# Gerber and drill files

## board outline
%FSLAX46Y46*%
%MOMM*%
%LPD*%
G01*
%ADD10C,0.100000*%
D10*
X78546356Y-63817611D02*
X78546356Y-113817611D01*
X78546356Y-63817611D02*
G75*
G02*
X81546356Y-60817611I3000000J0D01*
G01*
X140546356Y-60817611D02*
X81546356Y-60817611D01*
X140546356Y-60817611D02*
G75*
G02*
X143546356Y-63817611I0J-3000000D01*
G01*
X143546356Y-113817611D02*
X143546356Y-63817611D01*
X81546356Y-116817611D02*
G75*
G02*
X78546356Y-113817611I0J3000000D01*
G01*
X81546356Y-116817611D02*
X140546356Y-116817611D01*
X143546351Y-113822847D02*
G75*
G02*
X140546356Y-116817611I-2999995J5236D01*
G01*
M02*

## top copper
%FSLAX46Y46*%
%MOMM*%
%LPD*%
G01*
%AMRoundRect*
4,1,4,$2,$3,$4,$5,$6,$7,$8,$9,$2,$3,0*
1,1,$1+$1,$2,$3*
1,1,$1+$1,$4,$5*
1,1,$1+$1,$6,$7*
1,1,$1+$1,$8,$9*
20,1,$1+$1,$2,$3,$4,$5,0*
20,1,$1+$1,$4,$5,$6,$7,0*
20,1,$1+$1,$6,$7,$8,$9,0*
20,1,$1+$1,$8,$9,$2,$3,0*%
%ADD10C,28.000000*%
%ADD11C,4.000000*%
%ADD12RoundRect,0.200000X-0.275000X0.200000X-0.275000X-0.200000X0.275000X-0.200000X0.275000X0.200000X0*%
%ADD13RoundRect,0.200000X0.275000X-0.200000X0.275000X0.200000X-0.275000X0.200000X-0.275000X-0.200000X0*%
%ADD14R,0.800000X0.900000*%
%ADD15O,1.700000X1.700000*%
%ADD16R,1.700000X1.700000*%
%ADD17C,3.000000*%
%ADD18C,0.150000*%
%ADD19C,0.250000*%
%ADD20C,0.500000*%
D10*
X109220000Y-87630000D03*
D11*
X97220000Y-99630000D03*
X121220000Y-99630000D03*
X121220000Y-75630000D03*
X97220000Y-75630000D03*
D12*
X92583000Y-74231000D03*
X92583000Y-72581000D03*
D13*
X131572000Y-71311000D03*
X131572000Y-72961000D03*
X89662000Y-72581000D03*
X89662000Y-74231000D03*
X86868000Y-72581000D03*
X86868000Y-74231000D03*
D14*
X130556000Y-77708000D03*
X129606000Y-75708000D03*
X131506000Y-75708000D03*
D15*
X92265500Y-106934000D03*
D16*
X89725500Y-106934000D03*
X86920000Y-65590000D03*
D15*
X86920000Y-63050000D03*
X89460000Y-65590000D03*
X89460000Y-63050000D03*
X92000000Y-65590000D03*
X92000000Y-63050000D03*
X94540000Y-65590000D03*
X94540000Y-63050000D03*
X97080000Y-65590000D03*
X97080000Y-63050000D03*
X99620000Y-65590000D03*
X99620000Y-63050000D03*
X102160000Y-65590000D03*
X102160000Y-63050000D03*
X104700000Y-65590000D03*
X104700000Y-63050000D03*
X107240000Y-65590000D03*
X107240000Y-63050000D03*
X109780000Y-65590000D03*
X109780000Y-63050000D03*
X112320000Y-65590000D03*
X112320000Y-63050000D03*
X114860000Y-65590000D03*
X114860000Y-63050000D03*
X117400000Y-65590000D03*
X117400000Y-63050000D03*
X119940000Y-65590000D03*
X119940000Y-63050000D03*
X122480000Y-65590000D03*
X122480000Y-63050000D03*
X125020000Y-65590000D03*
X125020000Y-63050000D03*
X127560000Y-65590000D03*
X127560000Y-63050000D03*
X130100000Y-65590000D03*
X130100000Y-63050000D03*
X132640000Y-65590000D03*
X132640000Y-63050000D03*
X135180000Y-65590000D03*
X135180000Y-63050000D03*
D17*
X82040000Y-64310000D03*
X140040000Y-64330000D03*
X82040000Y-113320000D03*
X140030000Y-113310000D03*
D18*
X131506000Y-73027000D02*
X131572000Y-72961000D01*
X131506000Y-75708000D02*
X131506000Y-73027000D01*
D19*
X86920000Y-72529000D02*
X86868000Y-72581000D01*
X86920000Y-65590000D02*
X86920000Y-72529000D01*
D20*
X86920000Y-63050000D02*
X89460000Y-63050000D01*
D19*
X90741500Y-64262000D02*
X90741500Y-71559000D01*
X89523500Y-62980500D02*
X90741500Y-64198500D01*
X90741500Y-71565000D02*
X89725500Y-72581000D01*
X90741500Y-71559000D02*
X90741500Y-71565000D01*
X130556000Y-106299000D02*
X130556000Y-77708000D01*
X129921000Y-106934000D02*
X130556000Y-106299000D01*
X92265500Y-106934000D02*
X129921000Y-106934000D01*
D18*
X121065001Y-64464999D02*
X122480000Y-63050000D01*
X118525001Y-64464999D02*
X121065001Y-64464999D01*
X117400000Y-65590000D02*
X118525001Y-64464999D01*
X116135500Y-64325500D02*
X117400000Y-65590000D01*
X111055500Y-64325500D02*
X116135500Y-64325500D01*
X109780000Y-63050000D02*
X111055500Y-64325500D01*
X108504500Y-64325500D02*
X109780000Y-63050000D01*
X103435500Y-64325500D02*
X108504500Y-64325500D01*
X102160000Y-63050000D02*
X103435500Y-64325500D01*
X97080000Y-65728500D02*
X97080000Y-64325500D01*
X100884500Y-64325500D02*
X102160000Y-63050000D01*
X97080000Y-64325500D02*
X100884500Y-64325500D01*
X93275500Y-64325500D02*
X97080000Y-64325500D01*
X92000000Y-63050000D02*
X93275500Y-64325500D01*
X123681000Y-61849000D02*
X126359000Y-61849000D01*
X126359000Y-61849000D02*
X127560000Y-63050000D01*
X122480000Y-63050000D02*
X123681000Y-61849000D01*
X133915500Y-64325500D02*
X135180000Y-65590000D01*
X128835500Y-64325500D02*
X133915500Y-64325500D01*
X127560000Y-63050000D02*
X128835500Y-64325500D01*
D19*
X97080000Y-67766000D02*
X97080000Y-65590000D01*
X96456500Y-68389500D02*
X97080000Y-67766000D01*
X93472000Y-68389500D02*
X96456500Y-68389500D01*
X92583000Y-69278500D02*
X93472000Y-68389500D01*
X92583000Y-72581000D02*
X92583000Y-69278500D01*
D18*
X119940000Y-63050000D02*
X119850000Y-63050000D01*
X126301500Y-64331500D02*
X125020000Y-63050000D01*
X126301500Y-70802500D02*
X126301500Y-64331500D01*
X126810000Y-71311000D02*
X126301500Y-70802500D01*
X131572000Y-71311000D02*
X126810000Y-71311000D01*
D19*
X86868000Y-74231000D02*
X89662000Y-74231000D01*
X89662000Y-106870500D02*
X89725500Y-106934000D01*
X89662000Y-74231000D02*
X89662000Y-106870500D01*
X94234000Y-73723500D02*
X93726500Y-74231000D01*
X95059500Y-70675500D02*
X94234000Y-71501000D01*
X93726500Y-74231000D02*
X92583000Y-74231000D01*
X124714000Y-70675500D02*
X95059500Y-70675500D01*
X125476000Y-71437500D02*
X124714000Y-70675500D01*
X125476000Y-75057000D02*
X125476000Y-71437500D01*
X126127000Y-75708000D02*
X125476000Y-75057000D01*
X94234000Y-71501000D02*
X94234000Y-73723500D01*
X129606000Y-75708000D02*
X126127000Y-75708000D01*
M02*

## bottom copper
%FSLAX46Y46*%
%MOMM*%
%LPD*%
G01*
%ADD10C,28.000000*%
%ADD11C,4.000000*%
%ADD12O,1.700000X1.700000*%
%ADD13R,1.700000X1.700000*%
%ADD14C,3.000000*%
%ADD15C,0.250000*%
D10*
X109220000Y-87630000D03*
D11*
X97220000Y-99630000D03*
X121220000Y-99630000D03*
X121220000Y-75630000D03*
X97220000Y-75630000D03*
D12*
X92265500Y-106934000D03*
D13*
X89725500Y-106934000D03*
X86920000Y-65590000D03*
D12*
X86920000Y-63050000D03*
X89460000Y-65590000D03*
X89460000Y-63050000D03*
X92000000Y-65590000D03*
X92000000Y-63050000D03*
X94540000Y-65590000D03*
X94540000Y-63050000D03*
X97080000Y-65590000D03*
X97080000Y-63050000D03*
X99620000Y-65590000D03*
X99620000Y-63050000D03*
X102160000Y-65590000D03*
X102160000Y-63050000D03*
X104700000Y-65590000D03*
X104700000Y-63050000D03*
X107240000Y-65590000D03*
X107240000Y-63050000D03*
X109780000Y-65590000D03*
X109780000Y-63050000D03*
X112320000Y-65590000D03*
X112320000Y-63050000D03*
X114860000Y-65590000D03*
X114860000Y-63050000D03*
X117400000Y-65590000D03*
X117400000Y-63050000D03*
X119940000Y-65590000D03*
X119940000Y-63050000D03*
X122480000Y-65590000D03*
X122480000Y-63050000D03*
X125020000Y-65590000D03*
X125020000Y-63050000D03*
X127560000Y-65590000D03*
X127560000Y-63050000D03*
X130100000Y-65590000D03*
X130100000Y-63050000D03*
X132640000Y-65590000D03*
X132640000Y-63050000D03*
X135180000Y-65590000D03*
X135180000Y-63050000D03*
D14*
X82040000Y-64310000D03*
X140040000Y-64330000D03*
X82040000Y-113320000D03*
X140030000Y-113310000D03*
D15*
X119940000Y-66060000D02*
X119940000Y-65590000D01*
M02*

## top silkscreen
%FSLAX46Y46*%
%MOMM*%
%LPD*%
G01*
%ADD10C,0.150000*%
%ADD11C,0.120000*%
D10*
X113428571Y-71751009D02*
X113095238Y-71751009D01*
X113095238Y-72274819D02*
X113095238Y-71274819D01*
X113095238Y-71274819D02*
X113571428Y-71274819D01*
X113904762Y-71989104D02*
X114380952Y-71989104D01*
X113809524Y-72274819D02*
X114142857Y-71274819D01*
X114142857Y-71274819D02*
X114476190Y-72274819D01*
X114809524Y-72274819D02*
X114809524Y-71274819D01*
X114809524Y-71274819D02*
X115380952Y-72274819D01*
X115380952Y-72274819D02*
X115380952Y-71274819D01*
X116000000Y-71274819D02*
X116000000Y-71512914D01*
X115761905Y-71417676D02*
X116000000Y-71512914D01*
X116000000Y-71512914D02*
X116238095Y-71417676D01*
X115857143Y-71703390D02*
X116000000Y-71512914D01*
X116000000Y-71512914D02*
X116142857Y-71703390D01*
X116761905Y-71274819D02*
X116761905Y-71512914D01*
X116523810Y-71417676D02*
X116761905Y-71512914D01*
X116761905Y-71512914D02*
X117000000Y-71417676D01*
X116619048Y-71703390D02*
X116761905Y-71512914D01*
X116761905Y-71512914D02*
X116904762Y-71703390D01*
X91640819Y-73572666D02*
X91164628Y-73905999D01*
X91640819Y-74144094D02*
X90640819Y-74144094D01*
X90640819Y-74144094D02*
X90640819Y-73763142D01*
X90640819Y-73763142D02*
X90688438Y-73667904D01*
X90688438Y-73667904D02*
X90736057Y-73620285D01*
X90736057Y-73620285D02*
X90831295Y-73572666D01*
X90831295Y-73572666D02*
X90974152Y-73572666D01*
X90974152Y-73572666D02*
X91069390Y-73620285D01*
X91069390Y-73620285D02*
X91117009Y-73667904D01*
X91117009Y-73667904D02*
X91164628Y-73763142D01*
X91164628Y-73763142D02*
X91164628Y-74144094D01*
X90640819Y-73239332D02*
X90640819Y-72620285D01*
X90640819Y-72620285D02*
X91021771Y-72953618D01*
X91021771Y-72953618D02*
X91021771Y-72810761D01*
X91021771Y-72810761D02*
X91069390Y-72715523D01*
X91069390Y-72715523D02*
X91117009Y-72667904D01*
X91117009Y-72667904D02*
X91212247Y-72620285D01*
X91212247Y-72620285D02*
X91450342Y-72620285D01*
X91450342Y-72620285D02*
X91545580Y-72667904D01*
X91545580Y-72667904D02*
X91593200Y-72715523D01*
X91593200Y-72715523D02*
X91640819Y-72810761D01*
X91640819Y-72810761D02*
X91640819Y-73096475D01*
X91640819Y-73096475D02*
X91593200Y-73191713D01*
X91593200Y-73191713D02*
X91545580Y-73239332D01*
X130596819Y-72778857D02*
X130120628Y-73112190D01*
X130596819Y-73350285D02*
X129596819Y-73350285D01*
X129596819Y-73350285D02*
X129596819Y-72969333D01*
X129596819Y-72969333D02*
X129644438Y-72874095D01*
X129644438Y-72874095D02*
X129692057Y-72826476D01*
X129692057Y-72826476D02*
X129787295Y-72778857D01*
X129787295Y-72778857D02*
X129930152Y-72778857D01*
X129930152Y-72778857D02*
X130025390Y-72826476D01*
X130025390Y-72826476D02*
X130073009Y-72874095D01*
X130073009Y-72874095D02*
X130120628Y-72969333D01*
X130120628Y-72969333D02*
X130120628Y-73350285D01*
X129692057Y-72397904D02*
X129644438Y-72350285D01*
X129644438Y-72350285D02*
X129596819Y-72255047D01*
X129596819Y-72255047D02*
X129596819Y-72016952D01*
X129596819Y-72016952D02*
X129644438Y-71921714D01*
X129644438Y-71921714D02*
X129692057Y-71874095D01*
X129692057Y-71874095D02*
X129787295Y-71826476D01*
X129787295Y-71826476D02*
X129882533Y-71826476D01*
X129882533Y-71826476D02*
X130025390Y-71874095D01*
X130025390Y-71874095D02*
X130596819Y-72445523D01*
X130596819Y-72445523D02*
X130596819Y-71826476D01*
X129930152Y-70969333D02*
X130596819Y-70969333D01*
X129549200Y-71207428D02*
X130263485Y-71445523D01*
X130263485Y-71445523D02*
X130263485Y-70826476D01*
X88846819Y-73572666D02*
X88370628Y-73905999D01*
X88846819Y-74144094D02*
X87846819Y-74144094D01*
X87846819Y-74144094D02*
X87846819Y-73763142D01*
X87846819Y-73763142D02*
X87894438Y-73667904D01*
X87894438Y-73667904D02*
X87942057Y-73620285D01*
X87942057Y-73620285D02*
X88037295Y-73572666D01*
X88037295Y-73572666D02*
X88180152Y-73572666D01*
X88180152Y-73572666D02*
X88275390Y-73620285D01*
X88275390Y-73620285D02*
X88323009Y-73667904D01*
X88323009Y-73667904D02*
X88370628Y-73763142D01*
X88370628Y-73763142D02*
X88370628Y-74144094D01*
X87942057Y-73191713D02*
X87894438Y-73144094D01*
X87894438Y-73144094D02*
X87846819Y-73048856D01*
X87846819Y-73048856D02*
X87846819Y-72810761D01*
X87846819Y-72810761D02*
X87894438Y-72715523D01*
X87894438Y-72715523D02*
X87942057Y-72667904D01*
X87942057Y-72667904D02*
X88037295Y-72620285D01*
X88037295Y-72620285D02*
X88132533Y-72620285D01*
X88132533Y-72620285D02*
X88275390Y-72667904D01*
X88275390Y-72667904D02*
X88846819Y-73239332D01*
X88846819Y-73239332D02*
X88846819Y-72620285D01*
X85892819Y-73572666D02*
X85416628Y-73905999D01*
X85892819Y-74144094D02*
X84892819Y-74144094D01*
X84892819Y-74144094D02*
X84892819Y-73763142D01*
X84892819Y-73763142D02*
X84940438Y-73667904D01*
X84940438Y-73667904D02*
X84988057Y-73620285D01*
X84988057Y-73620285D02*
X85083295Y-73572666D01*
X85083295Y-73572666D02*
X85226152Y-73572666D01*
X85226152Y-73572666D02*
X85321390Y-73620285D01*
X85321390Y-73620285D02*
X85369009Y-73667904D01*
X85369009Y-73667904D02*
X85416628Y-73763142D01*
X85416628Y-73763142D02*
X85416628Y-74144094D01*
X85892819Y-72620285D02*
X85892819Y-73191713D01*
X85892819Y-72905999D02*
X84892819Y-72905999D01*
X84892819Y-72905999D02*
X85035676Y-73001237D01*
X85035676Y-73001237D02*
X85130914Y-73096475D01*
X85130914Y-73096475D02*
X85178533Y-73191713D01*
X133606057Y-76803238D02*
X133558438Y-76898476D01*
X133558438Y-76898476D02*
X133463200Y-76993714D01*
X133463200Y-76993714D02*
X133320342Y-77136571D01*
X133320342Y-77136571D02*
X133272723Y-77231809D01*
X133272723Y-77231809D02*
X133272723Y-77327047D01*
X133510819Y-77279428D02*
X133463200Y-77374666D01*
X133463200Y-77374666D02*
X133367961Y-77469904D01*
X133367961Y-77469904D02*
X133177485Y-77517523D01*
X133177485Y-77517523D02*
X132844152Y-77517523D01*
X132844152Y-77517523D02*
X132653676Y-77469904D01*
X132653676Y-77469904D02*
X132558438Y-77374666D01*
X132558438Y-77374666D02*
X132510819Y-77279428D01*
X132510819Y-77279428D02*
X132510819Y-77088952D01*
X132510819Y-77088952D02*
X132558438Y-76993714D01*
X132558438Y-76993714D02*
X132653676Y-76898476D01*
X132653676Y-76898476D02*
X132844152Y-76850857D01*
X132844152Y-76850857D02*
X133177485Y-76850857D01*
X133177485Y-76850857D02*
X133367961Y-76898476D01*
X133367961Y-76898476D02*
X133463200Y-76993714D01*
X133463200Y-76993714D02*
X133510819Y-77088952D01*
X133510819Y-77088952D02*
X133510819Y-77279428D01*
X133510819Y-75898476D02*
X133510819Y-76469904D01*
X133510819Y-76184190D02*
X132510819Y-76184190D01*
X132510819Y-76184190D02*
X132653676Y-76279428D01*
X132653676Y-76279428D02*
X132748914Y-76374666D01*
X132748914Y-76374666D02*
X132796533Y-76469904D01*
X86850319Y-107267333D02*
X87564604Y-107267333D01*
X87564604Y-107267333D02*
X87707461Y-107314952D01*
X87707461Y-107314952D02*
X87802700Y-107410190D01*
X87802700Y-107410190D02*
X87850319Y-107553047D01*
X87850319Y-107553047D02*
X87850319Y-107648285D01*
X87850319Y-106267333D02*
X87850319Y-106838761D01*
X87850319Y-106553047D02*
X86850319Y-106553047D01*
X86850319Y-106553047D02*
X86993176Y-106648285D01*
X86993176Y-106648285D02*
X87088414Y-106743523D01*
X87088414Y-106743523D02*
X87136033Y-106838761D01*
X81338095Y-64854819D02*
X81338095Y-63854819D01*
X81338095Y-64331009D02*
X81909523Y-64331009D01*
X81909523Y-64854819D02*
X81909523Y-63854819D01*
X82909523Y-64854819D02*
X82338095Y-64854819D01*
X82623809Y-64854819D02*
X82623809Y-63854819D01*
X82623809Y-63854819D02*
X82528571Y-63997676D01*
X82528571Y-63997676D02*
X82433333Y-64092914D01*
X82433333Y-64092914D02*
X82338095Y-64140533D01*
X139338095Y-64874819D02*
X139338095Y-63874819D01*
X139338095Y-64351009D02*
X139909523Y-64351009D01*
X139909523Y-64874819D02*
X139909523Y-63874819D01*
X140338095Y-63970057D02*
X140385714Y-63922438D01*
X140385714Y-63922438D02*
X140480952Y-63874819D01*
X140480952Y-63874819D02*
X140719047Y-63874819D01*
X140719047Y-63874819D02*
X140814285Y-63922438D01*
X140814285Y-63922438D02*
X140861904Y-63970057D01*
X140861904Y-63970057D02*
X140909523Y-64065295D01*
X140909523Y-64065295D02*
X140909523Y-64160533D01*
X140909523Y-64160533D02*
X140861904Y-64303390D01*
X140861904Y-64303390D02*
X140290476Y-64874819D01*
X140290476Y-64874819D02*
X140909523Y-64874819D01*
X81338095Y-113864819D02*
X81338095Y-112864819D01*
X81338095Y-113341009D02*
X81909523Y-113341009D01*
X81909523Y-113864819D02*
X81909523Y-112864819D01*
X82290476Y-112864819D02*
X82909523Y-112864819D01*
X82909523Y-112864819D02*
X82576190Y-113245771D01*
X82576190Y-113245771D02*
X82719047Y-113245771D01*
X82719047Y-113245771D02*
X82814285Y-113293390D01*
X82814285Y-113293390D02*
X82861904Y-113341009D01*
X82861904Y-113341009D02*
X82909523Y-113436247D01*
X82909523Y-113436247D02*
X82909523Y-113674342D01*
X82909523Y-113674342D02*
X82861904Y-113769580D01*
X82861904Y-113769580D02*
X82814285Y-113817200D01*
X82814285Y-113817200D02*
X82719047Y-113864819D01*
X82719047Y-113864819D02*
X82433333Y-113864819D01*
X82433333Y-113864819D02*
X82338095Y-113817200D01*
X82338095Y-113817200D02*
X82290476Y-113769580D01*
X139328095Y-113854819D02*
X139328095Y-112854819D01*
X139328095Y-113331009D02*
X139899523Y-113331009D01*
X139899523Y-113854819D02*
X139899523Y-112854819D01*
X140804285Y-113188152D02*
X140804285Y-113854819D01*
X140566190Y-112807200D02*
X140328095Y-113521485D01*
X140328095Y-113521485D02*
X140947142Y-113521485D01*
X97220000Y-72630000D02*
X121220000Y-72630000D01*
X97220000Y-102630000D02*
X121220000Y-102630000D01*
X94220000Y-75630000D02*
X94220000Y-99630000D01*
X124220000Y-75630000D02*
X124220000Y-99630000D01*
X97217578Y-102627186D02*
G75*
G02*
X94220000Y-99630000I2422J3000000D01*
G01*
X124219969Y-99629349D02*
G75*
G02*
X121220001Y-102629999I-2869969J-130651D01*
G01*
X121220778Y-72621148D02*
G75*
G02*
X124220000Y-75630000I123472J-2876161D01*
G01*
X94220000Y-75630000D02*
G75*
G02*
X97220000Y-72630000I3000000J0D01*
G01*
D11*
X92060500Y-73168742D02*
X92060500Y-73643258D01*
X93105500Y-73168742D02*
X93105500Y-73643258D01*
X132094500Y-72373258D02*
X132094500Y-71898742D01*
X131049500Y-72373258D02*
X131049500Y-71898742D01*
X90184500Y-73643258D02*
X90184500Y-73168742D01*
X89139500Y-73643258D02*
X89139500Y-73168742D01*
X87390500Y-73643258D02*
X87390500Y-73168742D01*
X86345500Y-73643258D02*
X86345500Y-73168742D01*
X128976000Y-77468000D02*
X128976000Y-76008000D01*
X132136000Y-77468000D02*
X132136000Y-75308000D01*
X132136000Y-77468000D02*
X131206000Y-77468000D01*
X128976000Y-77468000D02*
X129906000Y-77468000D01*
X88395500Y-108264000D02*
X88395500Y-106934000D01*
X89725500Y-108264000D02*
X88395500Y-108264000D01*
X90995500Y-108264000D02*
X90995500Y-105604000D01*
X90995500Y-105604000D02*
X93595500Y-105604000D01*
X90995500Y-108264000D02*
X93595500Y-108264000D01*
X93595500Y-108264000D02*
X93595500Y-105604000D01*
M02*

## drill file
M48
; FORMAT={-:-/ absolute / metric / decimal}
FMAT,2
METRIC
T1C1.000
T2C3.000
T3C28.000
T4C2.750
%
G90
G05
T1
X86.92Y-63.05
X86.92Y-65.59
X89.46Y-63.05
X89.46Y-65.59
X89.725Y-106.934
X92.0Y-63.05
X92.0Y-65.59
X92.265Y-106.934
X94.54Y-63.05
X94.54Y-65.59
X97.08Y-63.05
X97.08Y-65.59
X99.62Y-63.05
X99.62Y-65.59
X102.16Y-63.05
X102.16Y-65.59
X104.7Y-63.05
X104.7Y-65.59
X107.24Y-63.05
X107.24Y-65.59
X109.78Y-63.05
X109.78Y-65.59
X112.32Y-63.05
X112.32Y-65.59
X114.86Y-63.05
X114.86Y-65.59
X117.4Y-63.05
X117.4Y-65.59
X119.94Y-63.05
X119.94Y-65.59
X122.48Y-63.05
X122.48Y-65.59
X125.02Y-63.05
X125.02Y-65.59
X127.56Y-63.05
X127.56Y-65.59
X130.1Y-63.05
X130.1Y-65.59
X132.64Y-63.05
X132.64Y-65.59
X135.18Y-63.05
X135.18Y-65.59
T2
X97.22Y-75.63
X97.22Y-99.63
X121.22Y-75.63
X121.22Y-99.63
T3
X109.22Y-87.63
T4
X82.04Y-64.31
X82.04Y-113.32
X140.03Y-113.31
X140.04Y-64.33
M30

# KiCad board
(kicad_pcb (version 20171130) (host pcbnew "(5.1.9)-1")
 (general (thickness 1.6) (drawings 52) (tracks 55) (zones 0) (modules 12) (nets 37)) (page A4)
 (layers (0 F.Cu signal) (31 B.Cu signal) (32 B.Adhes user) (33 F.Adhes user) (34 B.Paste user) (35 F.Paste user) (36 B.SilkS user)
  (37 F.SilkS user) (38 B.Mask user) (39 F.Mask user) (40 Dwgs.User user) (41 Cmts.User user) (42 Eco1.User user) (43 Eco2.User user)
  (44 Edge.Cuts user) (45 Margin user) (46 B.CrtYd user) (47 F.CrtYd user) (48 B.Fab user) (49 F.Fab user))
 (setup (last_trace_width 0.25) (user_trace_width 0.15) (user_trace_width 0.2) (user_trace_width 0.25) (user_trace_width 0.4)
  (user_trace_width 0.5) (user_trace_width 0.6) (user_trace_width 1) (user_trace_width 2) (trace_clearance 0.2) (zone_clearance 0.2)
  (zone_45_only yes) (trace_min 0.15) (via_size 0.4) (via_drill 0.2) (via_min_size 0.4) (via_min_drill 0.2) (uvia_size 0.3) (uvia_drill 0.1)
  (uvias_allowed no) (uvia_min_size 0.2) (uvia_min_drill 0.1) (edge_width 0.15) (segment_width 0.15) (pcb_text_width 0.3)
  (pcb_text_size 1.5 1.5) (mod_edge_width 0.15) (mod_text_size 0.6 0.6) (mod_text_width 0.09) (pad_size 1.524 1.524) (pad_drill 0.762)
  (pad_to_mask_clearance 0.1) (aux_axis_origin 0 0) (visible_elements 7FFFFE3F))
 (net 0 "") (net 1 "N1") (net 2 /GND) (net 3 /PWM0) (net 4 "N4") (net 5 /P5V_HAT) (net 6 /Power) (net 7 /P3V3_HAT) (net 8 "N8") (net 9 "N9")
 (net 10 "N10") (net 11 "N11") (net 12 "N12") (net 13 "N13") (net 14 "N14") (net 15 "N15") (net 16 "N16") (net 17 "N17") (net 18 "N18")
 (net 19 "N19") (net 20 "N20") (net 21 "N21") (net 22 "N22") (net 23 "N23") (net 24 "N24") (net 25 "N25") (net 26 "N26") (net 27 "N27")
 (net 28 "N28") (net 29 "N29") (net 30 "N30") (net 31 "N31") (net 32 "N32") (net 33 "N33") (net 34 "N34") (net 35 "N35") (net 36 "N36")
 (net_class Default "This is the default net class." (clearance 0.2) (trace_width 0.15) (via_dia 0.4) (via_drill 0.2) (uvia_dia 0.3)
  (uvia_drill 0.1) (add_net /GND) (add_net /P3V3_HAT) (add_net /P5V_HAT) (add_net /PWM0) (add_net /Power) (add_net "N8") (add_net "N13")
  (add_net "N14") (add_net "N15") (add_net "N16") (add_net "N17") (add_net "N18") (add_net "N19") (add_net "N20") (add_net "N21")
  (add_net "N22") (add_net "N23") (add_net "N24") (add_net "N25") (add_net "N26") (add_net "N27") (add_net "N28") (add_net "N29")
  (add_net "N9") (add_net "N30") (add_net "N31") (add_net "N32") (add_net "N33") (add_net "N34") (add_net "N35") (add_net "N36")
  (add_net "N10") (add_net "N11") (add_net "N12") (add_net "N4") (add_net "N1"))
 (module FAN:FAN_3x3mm (layer F.Cu) (at 97.22 75.63)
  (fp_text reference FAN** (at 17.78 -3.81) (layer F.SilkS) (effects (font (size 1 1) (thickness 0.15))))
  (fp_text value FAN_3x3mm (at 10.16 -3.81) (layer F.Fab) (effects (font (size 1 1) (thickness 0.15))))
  (fp_line (start 0 -3) (end 24 -3) (layer F.SilkS) (width 0.15))
  (fp_line (start 0 27) (end 24 27) (layer F.SilkS) (width 0.15))
  (fp_line (start -3 0) (end -3 24) (layer F.SilkS) (width 0.15))
  (fp_line (start 27 0) (end 27 24) (layer F.SilkS) (width 0.15))
  (fp_arc (start 0 23.997186) (end -3 24) (angle -89.9) (layer F.SilkS) (width 0.15))
  (fp_arc (start 24.13 24.13) (end 24.000001 26.999999) (angle -95.2) (layer F.SilkS) (width 0.15))
  (fp_arc (start 24.12425 -0.132691) (end 27 0) (angle -95.1) (layer F.SilkS) (width 0.15))
  (fp_arc (start 0 0) (end 0 -3) (angle -90) (layer F.SilkS) (width 0.15))
  (pad 5 thru_hole circle (at 12 12) (size 28 28) (drill 28) (layers *.Cu *.Mask))
  (pad 4 thru_hole circle (at 0 24) (size 4 4) (drill 3) (layers *.Cu *.Mask))
  (pad 3 thru_hole circle (at 24 24) (size 4 4) (drill 3) (layers *.Cu *.Mask))
  (pad 2 thru_hole circle (at 24 0) (size 4 4) (drill 3) (layers *.Cu *.Mask))
  (pad 1 thru_hole circle (at 0 0) (size 4 4) (drill 3) (layers *.Cu *.Mask)))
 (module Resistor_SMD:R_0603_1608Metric (layer F.Cu) (at 92.583 73.406 270)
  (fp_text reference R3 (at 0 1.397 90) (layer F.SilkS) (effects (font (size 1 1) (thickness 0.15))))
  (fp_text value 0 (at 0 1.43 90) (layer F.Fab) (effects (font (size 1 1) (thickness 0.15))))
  (fp_line (start -0.237258 0.5225) (end 0.237258 0.5225) (layer F.SilkS) (width 0.12))
  (fp_line (start -0.237258 -0.5225) (end 0.237258 -0.5225) (layer F.SilkS) (width 0.12))
  (pad 2 smd roundrect (at 0.825 0 270) (size 0.8 0.95) (layers F.Cu F.Paste F.Mask) (roundrect_rratio 0.25) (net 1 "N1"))
  (pad 1 smd roundrect (at -0.825 0 270) (size 0.8 0.95) (layers F.Cu F.Paste F.Mask) (roundrect_rratio 0.25) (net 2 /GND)))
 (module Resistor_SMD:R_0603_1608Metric (layer F.Cu) (at 131.572 72.136 90)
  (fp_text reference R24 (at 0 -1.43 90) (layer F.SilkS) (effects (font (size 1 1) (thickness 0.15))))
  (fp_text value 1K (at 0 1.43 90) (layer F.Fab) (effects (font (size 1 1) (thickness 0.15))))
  (fp_line (start -0.237258 0.5225) (end 0.237258 0.5225) (layer F.SilkS) (width 0.12))
  (fp_line (start -0.237258 -0.5225) (end 0.237258 -0.5225) (layer F.SilkS) (width 0.12))
  (pad 2 smd roundrect (at 0.825 0 90) (size 0.8 0.95) (layers F.Cu F.Paste F.Mask) (roundrect_rratio 0.25) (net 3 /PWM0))
  (pad 1 smd roundrect (at -0.825 0 90) (size 0.8 0.95) (layers F.Cu F.Paste F.Mask) (roundrect_rratio 0.25) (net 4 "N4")))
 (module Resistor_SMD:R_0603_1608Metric (layer F.Cu) (at 89.662 73.406 90)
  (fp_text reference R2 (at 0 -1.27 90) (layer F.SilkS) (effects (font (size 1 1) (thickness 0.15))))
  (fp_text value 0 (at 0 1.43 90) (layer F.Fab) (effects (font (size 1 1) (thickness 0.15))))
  (fp_line (start -0.237258 0.5225) (end 0.237258 0.5225) (layer F.SilkS) (width 0.12))
  (fp_line (start -0.237258 -0.5225) (end 0.237258 -0.5225) (layer F.SilkS) (width 0.12))
  (pad 2 smd roundrect (at 0.825 0 90) (size 0.8 0.95) (layers F.Cu F.Paste F.Mask) (roundrect_rratio 0.25) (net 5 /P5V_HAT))
  (pad 1 smd roundrect (at -0.825 0 90) (size 0.8 0.95) (layers F.Cu F.Paste F.Mask) (roundrect_rratio 0.25) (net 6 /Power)))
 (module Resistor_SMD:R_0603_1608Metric (layer F.Cu) (at 86.868 73.406 90)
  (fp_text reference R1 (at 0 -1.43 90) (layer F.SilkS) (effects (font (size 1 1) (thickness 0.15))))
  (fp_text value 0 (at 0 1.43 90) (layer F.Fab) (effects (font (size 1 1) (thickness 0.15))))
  (fp_line (start -0.237258 0.5225) (end 0.237258 0.5225) (layer F.SilkS) (width 0.12))
  (fp_line (start -0.237258 -0.5225) (end 0.237258 -0.5225) (layer F.SilkS) (width 0.12))
  (pad 2 smd roundrect (at 0.825 0 90) (size 0.8 0.95) (layers F.Cu F.Paste F.Mask) (roundrect_rratio 0.25) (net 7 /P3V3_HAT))
  (pad 1 smd roundrect (at -0.825 0 90) (size 0.8 0.95) (layers F.Cu F.Paste F.Mask) (roundrect_rratio 0.25) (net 6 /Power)))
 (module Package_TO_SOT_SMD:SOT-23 (layer F.Cu) (at 130.556 76.708 270)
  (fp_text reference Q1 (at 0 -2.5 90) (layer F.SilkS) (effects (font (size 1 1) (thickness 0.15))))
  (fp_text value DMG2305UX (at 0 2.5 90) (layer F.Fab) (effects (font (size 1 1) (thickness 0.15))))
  (fp_line (start 0.76 1.58) (end -0.7 1.58) (layer F.SilkS) (width 0.12))
  (fp_line (start 0.76 -1.58) (end -1.4 -1.58) (layer F.SilkS) (width 0.12))
  (fp_line (start 0.76 -1.58) (end 0.76 -0.65) (layer F.SilkS) (width 0.12))
  (fp_line (start 0.76 1.58) (end 0.76 0.65) (layer F.SilkS) (width 0.12))
  (pad 3 smd rect (at 1 0 270) (size 0.9 0.8) (layers F.Cu F.Paste F.Mask) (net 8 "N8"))
  (pad 2 smd rect (at -1 0.95 270) (size 0.9 0.8) (layers F.Cu F.Paste F.Mask) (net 1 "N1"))
  (pad 1 smd rect (at -1 -0.95 270) (size 0.9 0.8) (layers F.Cu F.Paste F.Mask) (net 4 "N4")))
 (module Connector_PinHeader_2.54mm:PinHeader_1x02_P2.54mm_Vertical (layer F.Cu) (at 89.7255 106.934 90)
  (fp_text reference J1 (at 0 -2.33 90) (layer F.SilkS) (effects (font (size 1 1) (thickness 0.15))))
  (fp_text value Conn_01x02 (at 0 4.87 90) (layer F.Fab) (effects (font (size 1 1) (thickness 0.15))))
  (fp_line (start -1.33 -1.33) (end 0 -1.33) (layer F.SilkS) (width 0.12))
  (fp_line (start -1.33 0) (end -1.33 -1.33) (layer F.SilkS) (width 0.12))
  (fp_line (start -1.33 1.27) (end 1.33 1.27) (layer F.SilkS) (width 0.12))
  (fp_line (start 1.33 1.27) (end 1.33 3.87) (layer F.SilkS) (width 0.12))
  (fp_line (start -1.33 1.27) (end -1.33 3.87) (layer F.SilkS) (width 0.12))
  (fp_line (start -1.33 3.87) (end 1.33 3.87) (layer F.SilkS) (width 0.12))
  (pad 2 thru_hole oval (at 0 2.54 90) (size 1.7 1.7) (drill 1) (layers *.Cu *.Mask) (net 8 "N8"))
  (pad 1 thru_hole rect (at 0 0 90) (size 1.7 1.7) (drill 1) (layers *.Cu *.Mask) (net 6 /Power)))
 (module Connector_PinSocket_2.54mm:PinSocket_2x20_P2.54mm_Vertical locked (layer B.Cu) (at 86.92 65.59 270)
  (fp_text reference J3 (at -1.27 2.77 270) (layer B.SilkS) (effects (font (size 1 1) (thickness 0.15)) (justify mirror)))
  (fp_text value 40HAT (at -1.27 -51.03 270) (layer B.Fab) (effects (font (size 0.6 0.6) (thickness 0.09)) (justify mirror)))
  (pad 1 thru_hole rect (at 0 0 270) (size 1.7 1.7) (drill 1) (layers *.Cu *.Mask) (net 7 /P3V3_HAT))
  (pad 2 thru_hole oval (at -2.54 0 270) (size 1.7 1.7) (drill 1) (layers *.Cu *.Mask) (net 5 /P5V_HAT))
  (pad 3 thru_hole oval (at 0 -2.54 270) (size 1.7 1.7) (drill 1) (layers *.Cu *.Mask) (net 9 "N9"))
  (pad 4 thru_hole oval (at -2.54 -2.54 270) (size 1.7 1.7) (drill 1) (layers *.Cu *.Mask) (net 5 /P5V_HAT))
  (pad 5 thru_hole oval (at 0 -5.08 270) (size 1.7 1.7) (drill 1) (layers *.Cu *.Mask) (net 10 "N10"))
  (pad 6 thru_hole oval (at -2.54 -5.08 270) (size 1.7 1.7) (drill 1) (layers *.Cu *.Mask) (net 2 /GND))
  (pad 7 thru_hole oval (at 0 -7.62 270) (size 1.7 1.7) (drill 1) (layers *.Cu *.Mask) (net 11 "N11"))
  (pad 8 thru_hole oval (at -2.54 -7.62 270) (size 1.7 1.7) (drill 1) (layers *.Cu *.Mask) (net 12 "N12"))
  (pad 9 thru_hole oval (at 0 -10.16 270) (size 1.7 1.7) (drill 1) (layers *.Cu *.Mask) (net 2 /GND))
  (pad 10 thru_hole oval (at -2.54 -10.16 270) (size 1.7 1.7) (drill 1) (layers *.Cu *.Mask) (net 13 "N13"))
  (pad 11 thru_hole oval (at 0 -12.7 270) (size 1.7 1.7) (drill 1) (layers *.Cu *.Mask) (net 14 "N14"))
  (pad 12 thru_hole oval (at -2.54 -12.7 270) (size 1.7 1.7) (drill 1) (layers *.Cu *.Mask) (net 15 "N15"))
  (pad 13 thru_hole oval (at 0 -15.24 270) (size 1.7 1.7) (drill 1) (layers *.Cu *.Mask) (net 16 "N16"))
  (pad 14 thru_hole oval (at -2.54 -15.24 270) (size 1.7 1.7) (drill 1) (layers *.Cu *.Mask) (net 2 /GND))
  (pad 15 thru_hole oval (at 0 -17.78 270) (size 1.7 1.7) (drill 1) (layers *.Cu *.Mask) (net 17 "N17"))
  (pad 16 thru_hole oval (at -2.54 -17.78 270) (size 1.7 1.7) (drill 1) (layers *.Cu *.Mask) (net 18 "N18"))
  (pad 17 thru_hole oval (at 0 -20.32 270) (size 1.7 1.7) (drill 1) (layers *.Cu *.Mask) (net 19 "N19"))
  (pad 18 thru_hole oval (at -2.54 -20.32 270) (size 1.7 1.7) (drill 1) (layers *.Cu *.Mask) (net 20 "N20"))
  (pad 19 thru_hole oval (at 0 -22.86 270) (size 1.7 1.7) (drill 1) (layers *.Cu *.Mask) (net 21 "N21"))
  (pad 20 thru_hole oval (at -2.54 -22.86 270) (size 1.7 1.7) (drill 1) (layers *.Cu *.Mask) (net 2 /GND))
  (pad 21 thru_hole oval (at 0 -25.4 270) (size 1.7 1.7) (drill 1) (layers *.Cu *.Mask) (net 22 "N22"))
  (pad 22 thru_hole oval (at -2.54 -25.4 270) (size 1.7 1.7) (drill 1) (layers *.Cu *.Mask) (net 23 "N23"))
  (pad 23 thru_hole oval (at 0 -27.94 270) (size 1.7 1.7) (drill 1) (layers *.Cu *.Mask) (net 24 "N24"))
  (pad 24 thru_hole oval (at -2.54 -27.94 270) (size 1.7 1.7) (drill 1) (layers *.Cu *.Mask) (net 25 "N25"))
  (pad 25 thru_hole oval (at 0 -30.48 270) (size 1.7 1.7) (drill 1) (layers *.Cu *.Mask) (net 2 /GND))
  (pad 26 thru_hole oval (at -2.54 -30.48 270) (size 1.7 1.7) (drill 1) (layers *.Cu *.Mask) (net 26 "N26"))
  (pad 27 thru_hole oval (at 0 -33.02 270) (size 1.7 1.7) (drill 1) (layers *.Cu *.Mask) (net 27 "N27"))
  (pad 28 thru_hole oval (at -2.54 -33.02 270) (size 1.7 1.7) (drill 1) (layers *.Cu *.Mask) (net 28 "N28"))
  (pad 29 thru_hole oval (at 0 -35.56 270) (size 1.7 1.7) (drill 1) (layers *.Cu *.Mask) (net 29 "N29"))
  (pad 30 thru_hole oval (at -2.54 -35.56 270) (size 1.7 1.7) (drill 1) (layers *.Cu *.Mask) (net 2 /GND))
  (pad 31 thru_hole oval (at 0 -38.1 270) (size 1.7 1.7) (drill 1) (layers *.Cu *.Mask) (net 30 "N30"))
  (pad 32 thru_hole oval (at -2.54 -38.1 270) (size 1.7 1.7) (drill 1) (layers *.Cu *.Mask) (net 3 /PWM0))
  (pad 33 thru_hole oval (at 0 -40.64 270) (size 1.7 1.7) (drill 1) (layers *.Cu *.Mask) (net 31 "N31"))
  (pad 34 thru_hole oval (at -2.54 -40.64 270) (size 1.7 1.7) (drill 1) (layers *.Cu *.Mask) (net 2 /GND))
  (pad 35 thru_hole oval (at 0 -43.18 270) (size 1.7 1.7) (drill 1) (layers *.Cu *.Mask) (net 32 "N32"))
  (pad 36 thru_hole oval (at -2.54 -43.18 270) (size 1.7 1.7) (drill 1) (layers *.Cu *.Mask) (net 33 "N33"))
  (pad 37 thru_hole oval (at 0 -45.72 270) (size 1.7 1.7) (drill 1) (layers *.Cu *.Mask) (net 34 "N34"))
  (pad 38 thru_hole oval (at -2.54 -45.72 270) (size 1.7 1.7) (drill 1) (layers *.Cu *.Mask) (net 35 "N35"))
  (pad 39 thru_hole oval (at 0 -48.26 270) (size 1.7 1.7) (drill 1) (layers *.Cu *.Mask) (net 2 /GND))
  (pad 40 thru_hole oval (at -2.54 -48.26 270) (size 1.7 1.7) (drill 1) (layers *.Cu *.Mask) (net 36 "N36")))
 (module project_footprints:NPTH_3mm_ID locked (layer F.Cu) (at 82.04 64.31)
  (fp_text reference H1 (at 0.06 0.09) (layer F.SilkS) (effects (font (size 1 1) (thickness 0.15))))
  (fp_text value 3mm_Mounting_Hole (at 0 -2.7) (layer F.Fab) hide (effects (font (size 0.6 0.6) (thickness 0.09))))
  (pad "" np_thru_hole circle (at 0 0) (size 3 3) (drill 2.75) (layers *.Cu *.Mask) (clearance 1.6)))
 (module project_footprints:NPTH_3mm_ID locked (layer F.Cu) (at 140.04 64.33)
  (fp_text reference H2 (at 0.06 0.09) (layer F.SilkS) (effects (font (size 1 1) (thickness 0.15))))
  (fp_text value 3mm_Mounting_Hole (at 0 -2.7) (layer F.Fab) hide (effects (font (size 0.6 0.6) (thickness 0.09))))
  (pad "" np_thru_hole circle (at 0 0) (size 3 3) (drill 2.75) (layers *.Cu *.Mask) (clearance 1.6)))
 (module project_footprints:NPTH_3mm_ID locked (layer F.Cu) (at 82.04 113.32)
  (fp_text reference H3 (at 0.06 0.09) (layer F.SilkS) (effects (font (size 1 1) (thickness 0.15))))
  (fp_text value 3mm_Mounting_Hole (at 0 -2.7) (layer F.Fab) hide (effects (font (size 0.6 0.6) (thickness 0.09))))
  (pad "" np_thru_hole circle (at 0 0) (size 3 3) (drill 2.75) (layers *.Cu *.Mask) (clearance 1.6)))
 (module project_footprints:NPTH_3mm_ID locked (layer F.Cu) (at 140.03 113.31)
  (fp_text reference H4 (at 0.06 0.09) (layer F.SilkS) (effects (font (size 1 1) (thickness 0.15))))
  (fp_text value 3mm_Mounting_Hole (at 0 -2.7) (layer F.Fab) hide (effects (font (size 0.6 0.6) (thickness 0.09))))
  (pad "" np_thru_hole circle (at 0 0) (size 3 3) (drill 2.75) (layers *.Cu *.Mask) (clearance 1.6)))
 (gr_line (start 78.546356 63.817611) (end 78.546356 113.817611) (layer Edge.Cuts) (width 0.1))
 (gr_arc (start 81.546356 63.817611) (end 81.546356 60.817611) (angle -90) (layer Edge.Cuts) (width 0.1))
 (gr_line (start 140.546356 60.817611) (end 81.546356 60.817611) (layer Edge.Cuts) (width 0.1))
 (gr_arc (start 140.546356 63.817611) (end 143.546356 63.817611) (angle -90) (layer Edge.Cuts) (width 0.1))
 (gr_line (start 143.546356 113.817611) (end 143.546356 63.817611) (layer Edge.Cuts) (width 0.1))
 (gr_arc (start 81.546356 113.817611) (end 78.546356 113.817611) (angle -90) (layer Edge.Cuts) (width 0.1))
 (gr_line (start 81.546356 116.817611) (end 140.546356 116.817611) (layer Edge.Cuts) (width 0.1))
 (gr_arc (start 140.546356 113.817611) (end 140.546356 116.817611) (angle -89.9) (layer Edge.Cuts) (width 0.1))
 (segment (start 131.506 73.027) (end 131.572 72.961) (width 0.15) (layer F.Cu) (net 4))
 (segment (start 131.506 75.708) (end 131.506 73.027) (width 0.15) (layer F.Cu) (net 4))
 (segment (start 86.92 72.529) (end 86.868 72.581) (width 0.25) (layer F.Cu) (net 7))
 (segment (start 86.92 65.59) (end 86.92 72.529) (width 0.25) (layer F.Cu) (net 7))
 (segment (start 86.92 63.05) (end 89.46 63.05) (width 0.5) (layer F.Cu) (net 5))
 (segment (start 90.7415 64.262) (end 90.7415 71.559) (width 0.25) (layer F.Cu) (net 5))
 (segment (start 89.5235 62.9805) (end 90.7415 64.1985) (width 0.25) (layer F.Cu) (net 5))
 (segment (start 90.7415 71.565) (end 89.7255 72.581) (width 0.25) (layer F.Cu) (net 5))
 (segment (start 90.7415 71.559) (end 90.7415 71.565) (width 0.25) (layer F.Cu) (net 5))
 (segment (start 130.556 106.299) (end 130.556 77.708) (width 0.25) (layer F.Cu) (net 8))
 (segment (start 129.921 106.934) (end 130.556 106.299) (width 0.25) (layer F.Cu) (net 8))
 (segment (start 92.2655 106.934) (end 129.921 106.934) (width 0.25) (layer F.Cu) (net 8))
 (segment (start 121.065001 64.464999) (end 122.48 63.05) (width 0.15) (layer F.Cu) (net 2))
 (segment (start 118.525001 64.464999) (end 121.065001 64.464999) (width 0.15) (layer F.Cu) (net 2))
 (segment (start 117.4 65.59) (end 118.525001 64.464999) (width 0.15) (layer F.Cu) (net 2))
 (segment (start 116.1355 64.3255) (end 117.4 65.59) (width 0.15) (layer F.Cu) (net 2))
 (segment (start 111.0555 64.3255) (end 116.1355 64.3255) (width 0.15) (layer F.Cu) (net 2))
 (segment (start 109.78 63.05) (end 111.0555 64.3255) (width 0.15) (layer F.Cu) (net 2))
 (segment (start 108.5045 64.3255) (end 109.78 63.05) (width 0.15) (layer F.Cu) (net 2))
 (segment (start 103.4355 64.3255) (end 108.5045 64.3255) (width 0.15) (layer F.Cu) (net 2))
 (segment (start 102.16 63.05) (end 103.4355 64.3255) (width 0.15) (layer F.Cu) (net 2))
 (segment (start 97.08 65.7285) (end 97.08 64.3255) (width 0.15) (layer F.Cu) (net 2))
 (segment (start 100.8845 64.3255) (end 102.16 63.05) (width 0.15) (layer F.Cu) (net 2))
 (segment (start 97.08 64.3255) (end 100.8845 64.3255) (width 0.15) (layer F.Cu) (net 2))
 (segment (start 93.2755 64.3255) (end 97.08 64.3255) (width 0.15) (layer F.Cu) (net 2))
 (segment (start 92 63.05) (end 93.2755 64.3255) (width 0.15) (layer F.Cu) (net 2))
 (segment (start 123.681 61.849) (end 126.359 61.849) (width 0.15) (layer F.Cu) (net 2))
 (segment (start 126.359 61.849) (end 127.56 63.05) (width 0.15) (layer F.Cu) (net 2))
 (segment (start 122.48 63.05) (end 123.681 61.849) (width 0.15) (layer F.Cu) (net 2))
 (segment (start 133.9155 64.3255) (end 135.18 65.59) (width 0.15) (layer F.Cu) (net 2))
 (segment (start 128.8355 64.3255) (end 133.9155 64.3255) (width 0.15) (layer F.Cu) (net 2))
 (segment (start 127.56 63.05) (end 128.8355 64.3255) (width 0.15) (layer F.Cu) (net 2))
 (segment (start 97.08 67.766) (end 97.08 65.59) (width 0.25) (layer F.Cu) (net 2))
 (segment (start 96.4565 68.3895) (end 97.08 67.766) (width 0.25) (layer F.Cu) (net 2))
 (segment (start 93.472 68.3895) (end 96.4565 68.3895) (width 0.25) (layer F.Cu) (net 2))
 (segment (start 92.583 69.2785) (end 93.472 68.3895) (width 0.25) (layer F.Cu) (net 2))
 (segment (start 92.583 72.581) (end 92.583 69.2785) (width 0.25) (layer F.Cu) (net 2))
 (segment (start 119.94 66.06) (end 119.94 65.59) (width 0.25) (layer B.Cu) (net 27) (status 30))
 (segment (start 119.94 63.05) (end 119.85 63.05) (width 0.15) (layer F.Cu) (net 28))
 (segment (start 126.3015 64.3315) (end 125.02 63.05) (width 0.15) (layer F.Cu) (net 3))
 (segment (start 126.3015 70.8025) (end 126.3015 64.3315) (width 0.15) (layer F.Cu) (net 3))
 (segment (start 126.81 71.311) (end 126.3015 70.8025) (width 0.15) (layer F.Cu) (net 3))
 (segment (start 131.572 71.311) (end 126.81 71.311) (width 0.15) (layer F.Cu) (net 3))
 (segment (start 86.868 74.231) (end 89.662 74.231) (width 0.25) (layer F.Cu) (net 6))
 (segment (start 89.662 106.8705) (end 89.7255 106.934) (width 0.25) (layer F.Cu) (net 6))
 (segment (start 89.662 74.231) (end 89.662 106.8705) (width 0.25) (layer F.Cu) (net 6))
 (segment (start 94.234 73.7235) (end 93.7265 74.231) (width 0.25) (layer F.Cu) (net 1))
 (segment (start 95.0595 70.6755) (end 94.234 71.501) (width 0.25) (layer F.Cu) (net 1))
 (segment (start 93.7265 74.231) (end 92.583 74.231) (width 0.25) (layer F.Cu) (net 1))
 (segment (start 124.714 70.6755) (end 95.0595 70.6755) (width 0.25) (layer F.Cu) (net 1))
 (segment (start 125.476 71.4375) (end 124.714 70.6755) (width 0.25) (layer F.Cu) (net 1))
 (segment (start 125.476 75.057) (end 125.476 71.4375) (width 0.25) (layer F.Cu) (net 1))
 (segment (start 126.127 75.708) (end 125.476 75.057) (width 0.25) (layer F.Cu) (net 1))
 (segment (start 94.234 71.501) (end 94.234 73.7235) (width 0.25) (layer F.Cu) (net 1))
 (segment (start 129.606 75.708) (end 126.127 75.708) (width 0.25) (layer F.Cu) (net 1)))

